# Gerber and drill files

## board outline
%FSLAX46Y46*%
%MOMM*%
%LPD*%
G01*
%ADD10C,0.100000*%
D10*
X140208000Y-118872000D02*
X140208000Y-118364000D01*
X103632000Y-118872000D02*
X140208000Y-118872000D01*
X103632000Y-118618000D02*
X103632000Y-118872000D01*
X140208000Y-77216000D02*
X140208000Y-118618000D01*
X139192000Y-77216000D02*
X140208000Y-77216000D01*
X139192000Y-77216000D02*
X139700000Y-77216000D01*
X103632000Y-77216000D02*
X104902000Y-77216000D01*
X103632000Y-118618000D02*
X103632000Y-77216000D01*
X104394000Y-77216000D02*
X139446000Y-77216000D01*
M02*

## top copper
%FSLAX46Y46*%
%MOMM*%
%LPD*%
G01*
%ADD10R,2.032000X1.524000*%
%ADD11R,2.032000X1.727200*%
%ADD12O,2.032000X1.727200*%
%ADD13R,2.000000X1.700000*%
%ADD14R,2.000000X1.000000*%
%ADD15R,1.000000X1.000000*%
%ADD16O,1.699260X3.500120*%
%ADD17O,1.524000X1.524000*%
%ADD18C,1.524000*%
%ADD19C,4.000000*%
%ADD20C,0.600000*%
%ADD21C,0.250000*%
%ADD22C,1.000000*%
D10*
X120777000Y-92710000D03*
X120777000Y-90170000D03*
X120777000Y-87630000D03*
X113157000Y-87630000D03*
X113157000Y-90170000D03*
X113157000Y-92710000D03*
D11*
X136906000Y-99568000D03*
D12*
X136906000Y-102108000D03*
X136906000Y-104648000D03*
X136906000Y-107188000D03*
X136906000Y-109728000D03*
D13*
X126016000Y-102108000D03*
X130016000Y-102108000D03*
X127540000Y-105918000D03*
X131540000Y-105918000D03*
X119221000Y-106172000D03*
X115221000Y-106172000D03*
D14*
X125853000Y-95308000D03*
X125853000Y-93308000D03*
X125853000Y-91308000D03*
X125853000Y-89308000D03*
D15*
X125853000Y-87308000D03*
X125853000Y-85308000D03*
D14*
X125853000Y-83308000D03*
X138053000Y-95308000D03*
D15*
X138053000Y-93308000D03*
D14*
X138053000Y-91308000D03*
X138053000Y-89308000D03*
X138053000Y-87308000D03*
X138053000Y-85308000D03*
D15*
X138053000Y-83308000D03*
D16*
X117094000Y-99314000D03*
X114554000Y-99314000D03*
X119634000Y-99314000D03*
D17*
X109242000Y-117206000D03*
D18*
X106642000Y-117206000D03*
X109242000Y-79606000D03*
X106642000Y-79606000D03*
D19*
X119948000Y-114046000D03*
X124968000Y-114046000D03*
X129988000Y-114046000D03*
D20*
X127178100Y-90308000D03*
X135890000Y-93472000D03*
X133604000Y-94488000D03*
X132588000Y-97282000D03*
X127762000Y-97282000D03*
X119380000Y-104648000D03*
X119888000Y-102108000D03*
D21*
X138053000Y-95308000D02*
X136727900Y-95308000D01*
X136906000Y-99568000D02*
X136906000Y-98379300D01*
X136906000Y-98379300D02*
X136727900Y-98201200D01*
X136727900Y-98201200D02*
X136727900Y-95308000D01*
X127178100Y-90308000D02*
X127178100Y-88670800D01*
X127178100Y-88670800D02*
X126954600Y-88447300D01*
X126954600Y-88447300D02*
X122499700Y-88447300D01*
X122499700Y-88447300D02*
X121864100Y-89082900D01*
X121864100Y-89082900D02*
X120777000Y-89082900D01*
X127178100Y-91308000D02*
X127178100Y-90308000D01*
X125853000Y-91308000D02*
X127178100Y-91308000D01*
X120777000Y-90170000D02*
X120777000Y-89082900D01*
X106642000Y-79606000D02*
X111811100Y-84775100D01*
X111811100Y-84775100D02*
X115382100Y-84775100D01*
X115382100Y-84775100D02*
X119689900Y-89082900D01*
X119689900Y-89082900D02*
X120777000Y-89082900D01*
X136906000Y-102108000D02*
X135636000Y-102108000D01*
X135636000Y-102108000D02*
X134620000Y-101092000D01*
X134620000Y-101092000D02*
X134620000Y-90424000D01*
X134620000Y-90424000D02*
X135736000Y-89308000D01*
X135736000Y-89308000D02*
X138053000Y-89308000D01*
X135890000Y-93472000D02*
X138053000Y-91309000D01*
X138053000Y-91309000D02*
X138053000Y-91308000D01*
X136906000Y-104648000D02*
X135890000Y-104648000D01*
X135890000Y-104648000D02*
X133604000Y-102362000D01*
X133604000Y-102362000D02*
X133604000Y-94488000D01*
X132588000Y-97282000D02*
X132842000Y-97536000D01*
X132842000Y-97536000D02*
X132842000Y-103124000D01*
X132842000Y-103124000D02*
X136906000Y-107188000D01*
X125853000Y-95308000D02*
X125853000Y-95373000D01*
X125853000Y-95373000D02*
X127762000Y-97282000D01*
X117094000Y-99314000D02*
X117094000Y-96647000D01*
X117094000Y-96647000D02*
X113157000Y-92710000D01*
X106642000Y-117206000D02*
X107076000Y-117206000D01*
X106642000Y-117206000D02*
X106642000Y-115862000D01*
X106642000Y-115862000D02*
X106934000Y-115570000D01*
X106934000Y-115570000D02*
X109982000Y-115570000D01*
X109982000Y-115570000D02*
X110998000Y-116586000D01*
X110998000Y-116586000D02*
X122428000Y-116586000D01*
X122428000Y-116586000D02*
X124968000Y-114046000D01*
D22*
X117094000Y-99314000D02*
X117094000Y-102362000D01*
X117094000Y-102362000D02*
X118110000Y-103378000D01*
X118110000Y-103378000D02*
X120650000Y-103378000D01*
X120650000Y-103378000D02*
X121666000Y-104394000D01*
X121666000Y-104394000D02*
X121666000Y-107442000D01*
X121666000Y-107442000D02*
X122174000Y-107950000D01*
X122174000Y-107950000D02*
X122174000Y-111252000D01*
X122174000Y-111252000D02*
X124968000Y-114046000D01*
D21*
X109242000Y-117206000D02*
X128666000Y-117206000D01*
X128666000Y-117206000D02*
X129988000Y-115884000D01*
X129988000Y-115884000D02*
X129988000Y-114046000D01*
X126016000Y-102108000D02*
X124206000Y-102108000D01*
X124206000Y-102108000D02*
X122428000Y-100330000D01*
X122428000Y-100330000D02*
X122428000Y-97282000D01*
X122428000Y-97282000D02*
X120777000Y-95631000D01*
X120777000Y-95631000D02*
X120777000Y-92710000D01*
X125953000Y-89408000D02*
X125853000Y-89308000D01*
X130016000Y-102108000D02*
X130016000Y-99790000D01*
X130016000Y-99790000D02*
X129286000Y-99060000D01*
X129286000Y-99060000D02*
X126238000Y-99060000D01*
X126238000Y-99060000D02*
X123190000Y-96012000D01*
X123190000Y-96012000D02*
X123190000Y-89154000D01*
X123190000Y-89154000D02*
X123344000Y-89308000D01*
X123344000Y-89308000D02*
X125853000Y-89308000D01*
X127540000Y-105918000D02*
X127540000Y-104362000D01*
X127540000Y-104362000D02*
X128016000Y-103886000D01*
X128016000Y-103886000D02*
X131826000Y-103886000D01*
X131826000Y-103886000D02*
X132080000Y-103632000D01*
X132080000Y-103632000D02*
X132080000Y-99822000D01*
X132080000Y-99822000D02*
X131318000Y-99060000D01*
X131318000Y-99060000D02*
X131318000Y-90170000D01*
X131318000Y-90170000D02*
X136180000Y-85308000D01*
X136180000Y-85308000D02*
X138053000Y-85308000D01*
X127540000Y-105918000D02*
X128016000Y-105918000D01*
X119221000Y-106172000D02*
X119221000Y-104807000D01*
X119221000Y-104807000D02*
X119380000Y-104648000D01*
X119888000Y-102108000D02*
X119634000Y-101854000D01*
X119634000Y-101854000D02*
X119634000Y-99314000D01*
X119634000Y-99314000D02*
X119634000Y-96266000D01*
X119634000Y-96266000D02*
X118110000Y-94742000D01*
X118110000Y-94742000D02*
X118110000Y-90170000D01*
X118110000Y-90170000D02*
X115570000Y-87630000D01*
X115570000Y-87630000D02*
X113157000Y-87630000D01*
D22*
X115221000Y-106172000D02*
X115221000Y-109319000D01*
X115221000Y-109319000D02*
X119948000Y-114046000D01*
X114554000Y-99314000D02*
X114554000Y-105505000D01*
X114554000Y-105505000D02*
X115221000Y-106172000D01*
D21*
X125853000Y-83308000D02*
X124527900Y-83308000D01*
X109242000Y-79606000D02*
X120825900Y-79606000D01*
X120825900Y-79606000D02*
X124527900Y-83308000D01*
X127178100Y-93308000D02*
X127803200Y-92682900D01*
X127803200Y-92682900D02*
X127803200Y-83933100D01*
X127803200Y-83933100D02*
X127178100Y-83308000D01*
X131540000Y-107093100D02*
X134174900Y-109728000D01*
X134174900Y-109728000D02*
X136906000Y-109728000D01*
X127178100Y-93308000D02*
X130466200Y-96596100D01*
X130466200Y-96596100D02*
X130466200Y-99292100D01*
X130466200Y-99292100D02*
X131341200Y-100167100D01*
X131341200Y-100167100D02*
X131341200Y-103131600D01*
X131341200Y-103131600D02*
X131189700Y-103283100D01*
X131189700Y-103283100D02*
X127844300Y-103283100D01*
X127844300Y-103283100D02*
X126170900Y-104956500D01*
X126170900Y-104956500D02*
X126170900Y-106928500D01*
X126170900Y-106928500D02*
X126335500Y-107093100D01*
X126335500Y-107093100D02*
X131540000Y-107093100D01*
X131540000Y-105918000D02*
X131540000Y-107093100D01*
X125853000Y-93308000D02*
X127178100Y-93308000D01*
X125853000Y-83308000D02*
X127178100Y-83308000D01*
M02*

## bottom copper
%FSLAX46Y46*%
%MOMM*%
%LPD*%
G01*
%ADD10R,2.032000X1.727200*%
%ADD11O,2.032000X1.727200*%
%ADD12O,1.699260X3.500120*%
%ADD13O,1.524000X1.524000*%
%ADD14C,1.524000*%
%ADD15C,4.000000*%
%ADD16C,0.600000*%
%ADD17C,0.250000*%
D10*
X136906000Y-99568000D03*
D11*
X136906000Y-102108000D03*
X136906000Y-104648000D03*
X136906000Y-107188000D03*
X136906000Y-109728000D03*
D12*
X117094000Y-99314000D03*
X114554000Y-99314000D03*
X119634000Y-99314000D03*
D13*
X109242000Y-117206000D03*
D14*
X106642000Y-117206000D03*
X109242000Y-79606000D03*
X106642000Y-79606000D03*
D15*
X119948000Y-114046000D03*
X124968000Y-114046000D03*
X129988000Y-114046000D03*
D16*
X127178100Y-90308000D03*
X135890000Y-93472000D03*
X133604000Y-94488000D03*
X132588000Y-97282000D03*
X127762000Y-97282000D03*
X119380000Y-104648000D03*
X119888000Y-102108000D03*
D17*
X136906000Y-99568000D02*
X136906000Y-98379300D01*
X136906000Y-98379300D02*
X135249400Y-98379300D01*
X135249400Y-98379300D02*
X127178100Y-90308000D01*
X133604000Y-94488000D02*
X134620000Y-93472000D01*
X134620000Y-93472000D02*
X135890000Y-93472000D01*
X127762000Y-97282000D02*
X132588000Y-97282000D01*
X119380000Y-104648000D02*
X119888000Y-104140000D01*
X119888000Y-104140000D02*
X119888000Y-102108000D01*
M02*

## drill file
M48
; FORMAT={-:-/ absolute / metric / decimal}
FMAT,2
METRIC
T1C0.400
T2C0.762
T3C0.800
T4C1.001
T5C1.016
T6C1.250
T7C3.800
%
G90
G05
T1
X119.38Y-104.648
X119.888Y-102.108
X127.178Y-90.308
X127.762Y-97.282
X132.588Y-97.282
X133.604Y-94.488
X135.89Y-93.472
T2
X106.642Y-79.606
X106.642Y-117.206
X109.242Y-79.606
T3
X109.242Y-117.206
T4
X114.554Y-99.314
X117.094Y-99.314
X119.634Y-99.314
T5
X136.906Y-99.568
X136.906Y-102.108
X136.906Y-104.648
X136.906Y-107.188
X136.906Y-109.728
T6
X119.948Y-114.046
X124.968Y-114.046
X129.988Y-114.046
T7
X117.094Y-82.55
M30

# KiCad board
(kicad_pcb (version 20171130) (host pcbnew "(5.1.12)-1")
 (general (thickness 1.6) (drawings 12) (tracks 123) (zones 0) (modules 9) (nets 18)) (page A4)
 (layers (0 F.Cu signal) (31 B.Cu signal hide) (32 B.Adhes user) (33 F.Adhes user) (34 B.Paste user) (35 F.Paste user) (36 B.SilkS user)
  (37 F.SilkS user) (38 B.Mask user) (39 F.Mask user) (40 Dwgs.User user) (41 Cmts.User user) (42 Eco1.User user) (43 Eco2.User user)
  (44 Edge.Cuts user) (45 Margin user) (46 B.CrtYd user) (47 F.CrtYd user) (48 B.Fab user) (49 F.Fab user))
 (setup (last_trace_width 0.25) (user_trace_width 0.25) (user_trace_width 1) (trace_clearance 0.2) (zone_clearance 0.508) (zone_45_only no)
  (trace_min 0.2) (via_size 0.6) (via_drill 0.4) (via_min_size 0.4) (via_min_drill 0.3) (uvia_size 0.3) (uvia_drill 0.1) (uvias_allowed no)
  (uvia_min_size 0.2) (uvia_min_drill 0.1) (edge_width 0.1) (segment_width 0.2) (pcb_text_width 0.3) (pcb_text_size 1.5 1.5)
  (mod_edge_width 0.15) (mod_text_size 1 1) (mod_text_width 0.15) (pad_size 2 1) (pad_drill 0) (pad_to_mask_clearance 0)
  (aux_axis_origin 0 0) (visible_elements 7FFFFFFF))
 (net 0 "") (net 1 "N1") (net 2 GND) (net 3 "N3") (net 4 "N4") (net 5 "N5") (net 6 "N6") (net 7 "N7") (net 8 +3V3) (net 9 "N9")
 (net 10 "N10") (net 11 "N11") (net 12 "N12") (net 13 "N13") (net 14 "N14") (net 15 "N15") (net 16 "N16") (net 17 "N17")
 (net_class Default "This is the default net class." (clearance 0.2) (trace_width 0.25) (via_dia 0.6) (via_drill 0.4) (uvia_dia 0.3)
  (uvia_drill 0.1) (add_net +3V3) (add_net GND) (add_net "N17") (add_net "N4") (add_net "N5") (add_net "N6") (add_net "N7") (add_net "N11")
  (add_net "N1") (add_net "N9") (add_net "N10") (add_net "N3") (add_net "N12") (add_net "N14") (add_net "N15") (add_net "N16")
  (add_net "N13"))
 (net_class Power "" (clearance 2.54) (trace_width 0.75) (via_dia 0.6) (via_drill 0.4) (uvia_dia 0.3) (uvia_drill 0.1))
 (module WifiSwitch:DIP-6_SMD (layer F.Cu) (at 116.967 88.9 90)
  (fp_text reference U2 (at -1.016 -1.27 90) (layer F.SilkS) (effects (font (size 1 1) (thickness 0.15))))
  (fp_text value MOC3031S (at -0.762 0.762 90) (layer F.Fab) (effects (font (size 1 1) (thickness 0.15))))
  (pad 1 smd rect (at -3.81 3.81 90) (size 1.524 2.032) (layers F.Cu F.Paste F.Mask) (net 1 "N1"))
  (pad 2 smd rect (at -1.27 3.81 90) (size 1.524 2.032) (layers F.Cu F.Paste F.Mask) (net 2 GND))
  (pad 3 smd rect (at 1.27 3.81 90) (size 1.524 2.032) (layers F.Cu F.Paste F.Mask))
  (pad 4 smd rect (at 1.27 -3.81 90) (size 1.524 2.032) (layers F.Cu F.Paste F.Mask) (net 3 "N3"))
  (pad 5 smd rect (at -1.27 -3.81 90) (size 1.524 2.032) (layers F.Cu F.Paste F.Mask))
  (pad 6 smd rect (at -3.81 -3.81 90) (size 1.524 2.032) (layers F.Cu F.Paste F.Mask) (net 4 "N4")))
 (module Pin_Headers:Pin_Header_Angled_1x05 (layer F.Cu) (at 136.906 99.568)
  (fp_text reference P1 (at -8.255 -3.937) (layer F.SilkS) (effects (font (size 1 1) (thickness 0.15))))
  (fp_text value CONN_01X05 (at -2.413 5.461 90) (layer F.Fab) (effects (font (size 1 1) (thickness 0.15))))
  (pad 1 thru_hole rect (at 0 0) (size 2.032 1.7272) (drill 1.016) (layers *.Cu *.Mask F.SilkS) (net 2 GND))
  (pad 2 thru_hole oval (at 0 2.54) (size 2.032 1.7272) (drill 1.016) (layers *.Cu *.Mask F.SilkS) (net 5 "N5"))
  (pad 3 thru_hole oval (at 0 5.08) (size 2.032 1.7272) (drill 1.016) (layers *.Cu *.Mask F.SilkS) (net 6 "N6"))
  (pad 4 thru_hole oval (at 0 7.62) (size 2.032 1.7272) (drill 1.016) (layers *.Cu *.Mask F.SilkS) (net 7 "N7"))
  (pad 5 thru_hole oval (at 0 10.16) (size 2.032 1.7272) (drill 1.016) (layers *.Cu *.Mask F.SilkS) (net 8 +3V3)))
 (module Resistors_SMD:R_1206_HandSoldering (layer F.Cu) (at 128.016 102.108)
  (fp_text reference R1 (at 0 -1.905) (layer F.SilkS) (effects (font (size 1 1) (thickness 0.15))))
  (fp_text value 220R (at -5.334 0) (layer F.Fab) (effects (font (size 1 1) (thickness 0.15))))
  (pad 1 smd rect (at -2 0) (size 2 1.7) (layers F.Cu F.Paste F.Mask) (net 1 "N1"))
  (pad 2 smd rect (at 2 0) (size 2 1.7) (layers F.Cu F.Paste F.Mask) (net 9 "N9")))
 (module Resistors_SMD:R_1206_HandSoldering (layer F.Cu) (at 129.54 105.918)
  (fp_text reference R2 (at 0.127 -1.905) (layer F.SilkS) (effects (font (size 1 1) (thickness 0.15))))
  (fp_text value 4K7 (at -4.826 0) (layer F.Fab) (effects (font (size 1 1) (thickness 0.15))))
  (pad 1 smd rect (at -2 0) (size 2 1.7) (layers F.Cu F.Paste F.Mask) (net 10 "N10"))
  (pad 2 smd rect (at 2 0) (size 2 1.7) (layers F.Cu F.Paste F.Mask) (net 8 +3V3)))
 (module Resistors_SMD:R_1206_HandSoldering (layer F.Cu) (at 117.221 106.172 180)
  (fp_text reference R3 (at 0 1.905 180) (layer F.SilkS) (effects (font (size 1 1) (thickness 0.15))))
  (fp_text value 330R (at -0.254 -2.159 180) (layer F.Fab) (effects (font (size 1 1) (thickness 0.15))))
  (pad 1 smd rect (at -2 0 180) (size 2 1.7) (layers F.Cu F.Paste F.Mask) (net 3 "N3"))
  (pad 2 smd rect (at 2 0 180) (size 2 1.7) (layers F.Cu F.Paste F.Mask) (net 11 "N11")))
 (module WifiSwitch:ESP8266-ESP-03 (layer F.Cu) (at 131.953 89.408)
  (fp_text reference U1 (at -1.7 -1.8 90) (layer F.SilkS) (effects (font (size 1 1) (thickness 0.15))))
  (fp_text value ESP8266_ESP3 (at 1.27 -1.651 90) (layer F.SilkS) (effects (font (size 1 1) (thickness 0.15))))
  (pad 14 smd rect (at -6.1 5.9) (size 2 1) (layers F.Cu F.Paste F.Mask) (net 7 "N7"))
  (pad 13 smd rect (at -6.1 3.9) (size 2 1) (layers F.Cu F.Paste F.Mask) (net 8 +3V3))
  (pad 12 smd rect (at -6.1 1.9) (size 2 1) (layers F.Cu F.Paste F.Mask) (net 2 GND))
  (pad 11 smd rect (at -6.1 -0.1) (size 2 1) (layers F.Cu F.Paste F.Mask) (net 9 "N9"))
  (pad 10 smd rect (at -6.1 -2.1) (size 1 1) (layers F.Cu F.Paste F.Mask) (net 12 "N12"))
  (pad 9 smd rect (at -6.1 -4.1) (size 1 1) (layers F.Cu F.Paste F.Mask) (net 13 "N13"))
  (pad 8 smd rect (at -6.1 -6.1) (size 2 1) (layers F.Cu F.Paste F.Mask) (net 8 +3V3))
  (pad 1 smd rect (at 6.1 5.9) (size 2 1) (layers F.Cu F.Paste F.Mask) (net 2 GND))
  (pad 2 smd rect (at 6.1 3.9) (size 1 1) (layers F.Cu F.Paste F.Mask) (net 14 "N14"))
  (pad 3 smd rect (at 6.1 1.9) (size 2 1) (layers F.Cu F.Paste F.Mask) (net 6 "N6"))
  (pad 4 smd rect (at 6.1 -0.1) (size 2 1) (layers F.Cu F.Paste F.Mask) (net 5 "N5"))
  (pad 5 smd rect (at 6.1 -2.1) (size 2 1) (layers F.Cu F.Paste F.Mask) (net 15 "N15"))
  (pad 6 smd rect (at 6.1 -4.1) (size 2 1) (layers F.Cu F.Paste F.Mask) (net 10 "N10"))
  (pad 7 smd rect (at 6.1 -6.1) (size 1 1) (layers F.Cu F.Paste F.Mask) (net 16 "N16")))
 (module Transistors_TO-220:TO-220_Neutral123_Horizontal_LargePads (layer F.Cu) (at 117.094 99.314)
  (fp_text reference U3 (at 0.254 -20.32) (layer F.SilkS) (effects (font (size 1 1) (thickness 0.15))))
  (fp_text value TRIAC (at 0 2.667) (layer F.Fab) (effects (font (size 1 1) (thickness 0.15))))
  (pad 2 thru_hole oval (at 0 0 90) (size 3.50012 1.69926) (drill 1.00076) (layers *.Cu *.Mask F.SilkS) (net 4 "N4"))
  (pad 1 thru_hole oval (at -2.54 0 90) (size 3.50012 1.69926) (drill 1.00076) (layers *.Cu *.Mask F.SilkS) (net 11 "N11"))
  (pad 3 thru_hole oval (at 2.54 0 90) (size 3.50012 1.69926) (drill 1.00076) (layers *.Cu *.Mask F.SilkS) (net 3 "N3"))
  (pad "" np_thru_hole circle (at 0 -16.764 90) (size 3.79984 3.79984) (drill 3.79984) (layers *.Cu *.Mask F.SilkS)))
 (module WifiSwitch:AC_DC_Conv (layer F.Cu) (at 107.442 98.806 270)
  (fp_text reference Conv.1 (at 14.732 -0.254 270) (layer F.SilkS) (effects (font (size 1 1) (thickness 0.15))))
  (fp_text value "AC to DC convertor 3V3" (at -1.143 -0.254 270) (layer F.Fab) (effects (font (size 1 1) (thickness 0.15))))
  (pad 3 thru_hole oval (at 18.4 -1.8 270) (size 1.524 1.524) (drill 0.8) (layers *.Cu *.Mask F.SilkS) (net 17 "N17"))
  (pad 4 thru_hole circle (at 18.4 0.8 270) (size 1.524 1.524) (drill 0.762) (layers *.Cu *.Mask F.SilkS) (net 4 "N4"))
  (pad 1 thru_hole circle (at -19.2 -1.8 270) (size 1.524 1.524) (drill 0.762) (layers *.Cu *.Mask F.SilkS) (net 8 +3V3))
  (pad 2 thru_hole circle (at -19.2 0.8 270) (size 1.524 1.524) (drill 0.762) (layers *.Cu *.Mask F.SilkS) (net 2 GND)))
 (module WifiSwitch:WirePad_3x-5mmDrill (layer F.Cu) (at 124.968 114.046)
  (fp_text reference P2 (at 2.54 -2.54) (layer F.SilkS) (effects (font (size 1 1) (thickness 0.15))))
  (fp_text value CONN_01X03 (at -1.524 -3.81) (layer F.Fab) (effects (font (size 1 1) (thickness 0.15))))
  (pad 1 thru_hole circle (at -5.02 0) (size 4 4) (drill 1.25) (layers *.Cu *.Mask F.SilkS) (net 11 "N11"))
  (pad 2 thru_hole circle (at 0 0) (size 4 4) (drill 1.25) (layers *.Cu *.Mask F.SilkS) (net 4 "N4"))
  (pad 3 thru_hole circle (at 5.02 0) (size 4 4) (drill 1.25) (layers *.Cu *.Mask F.SilkS) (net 17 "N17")))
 (gr_line (start 140.208 118.872) (end 140.208 118.364) (angle 90) (layer Edge.Cuts) (width 0.1))
 (gr_line (start 103.632 118.872) (end 140.208 118.872) (angle 90) (layer Edge.Cuts) (width 0.1))
 (gr_line (start 103.632 118.618) (end 103.632 118.872) (angle 90) (layer Edge.Cuts) (width 0.1))
 (gr_line (start 140.208 77.216) (end 140.208 118.618) (angle 90) (layer Edge.Cuts) (width 0.1))
 (gr_line (start 139.192 77.216) (end 140.208 77.216) (angle 90) (layer Edge.Cuts) (width 0.1))
 (gr_line (start 139.192 77.216) (end 139.7 77.216) (angle 90) (layer Edge.Cuts) (width 0.1))
 (gr_line (start 103.632 77.216) (end 104.902 77.216) (angle 90) (layer Edge.Cuts) (width 0.1))
 (gr_line (start 103.632 118.618) (end 103.632 77.216) (angle 90) (layer Edge.Cuts) (width 0.1))
 (gr_line (start 104.394 77.216) (end 139.446 77.216) (angle 90) (layer Edge.Cuts) (width 0.1))
 (segment (start 138.053 95.308) (end 136.7279 95.308) (width 0.25) (layer F.Cu) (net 2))
 (segment (start 136.906 99.568) (end 136.906 98.3793) (width 0.25) (layer F.Cu) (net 2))
 (segment (start 136.906 98.3793) (end 136.7279 98.2012) (width 0.25) (layer F.Cu) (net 2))
 (segment (start 136.7279 98.2012) (end 136.7279 95.308) (width 0.25) (layer F.Cu) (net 2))
 (segment (start 136.906 99.568) (end 136.906 98.3793) (width 0.25) (layer B.Cu) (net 2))
 (segment (start 127.1781 90.308) (end 127.1781 88.6708) (width 0.25) (layer F.Cu) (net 2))
 (segment (start 127.1781 88.6708) (end 126.9546 88.4473) (width 0.25) (layer F.Cu) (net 2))
 (segment (start 126.9546 88.4473) (end 122.4997 88.4473) (width 0.25) (layer F.Cu) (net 2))
 (segment (start 122.4997 88.4473) (end 121.8641 89.0829) (width 0.25) (layer F.Cu) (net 2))
 (segment (start 121.8641 89.0829) (end 120.777 89.0829) (width 0.25) (layer F.Cu) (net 2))
 (segment (start 127.1781 91.308) (end 127.1781 90.308) (width 0.25) (layer F.Cu) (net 2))
 (segment (start 136.906 98.3793) (end 135.2494 98.3793) (width 0.25) (layer B.Cu) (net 2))
 (segment (start 135.2494 98.3793) (end 127.1781 90.308) (width 0.25) (layer B.Cu) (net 2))
 (segment (start 125.853 91.308) (end 127.1781 91.308) (width 0.25) (layer F.Cu) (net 2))
 (segment (start 120.777 90.17) (end 120.777 89.0829) (width 0.25) (layer F.Cu) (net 2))
 (segment (start 106.642 79.606) (end 111.8111 84.7751) (width 0.25) (layer F.Cu) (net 2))
 (segment (start 111.8111 84.7751) (end 115.3821 84.7751) (width 0.25) (layer F.Cu) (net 2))
 (segment (start 115.3821 84.7751) (end 119.6899 89.0829) (width 0.25) (layer F.Cu) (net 2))
 (segment (start 119.6899 89.0829) (end 120.777 89.0829) (width 0.25) (layer F.Cu) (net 2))
 (via (at 127.1781 90.308) (size 0.6) (layers F.Cu B.Cu) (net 2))
 (segment (start 136.906 102.108) (end 135.636 102.108) (width 0.25) (layer F.Cu) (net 5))
 (segment (start 135.636 102.108) (end 134.62 101.092) (width 0.25) (layer F.Cu) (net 5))
 (segment (start 134.62 101.092) (end 134.62 90.424) (width 0.25) (layer F.Cu) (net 5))
 (segment (start 134.62 90.424) (end 135.736 89.308) (width 0.25) (layer F.Cu) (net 5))
 (segment (start 135.736 89.308) (end 138.053 89.308) (width 0.25) (layer F.Cu) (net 5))
 (segment (start 135.89 93.472) (end 138.053 91.309) (width 0.25) (layer F.Cu) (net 6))
 (segment (start 138.053 91.309) (end 138.053 91.308) (width 0.25) (layer F.Cu) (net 6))
 (segment (start 133.604 94.488) (end 134.62 93.472) (width 0.25) (layer B.Cu) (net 6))
 (segment (start 134.62 93.472) (end 135.89 93.472) (width 0.25) (layer B.Cu) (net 6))
 (segment (start 136.906 104.648) (end 135.89 104.648) (width 0.25) (layer F.Cu) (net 6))
 (segment (start 135.89 104.648) (end 133.604 102.362) (width 0.25) (layer F.Cu) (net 6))
 (segment (start 133.604 102.362) (end 133.604 94.488) (width 0.25) (layer F.Cu) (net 6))
 (via (at 135.89 93.472) (size 0.6) (layers F.Cu B.Cu) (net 6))
 (via (at 133.604 94.488) (size 0.6) (layers F.Cu B.Cu) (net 6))
 (segment (start 132.588 97.282) (end 132.842 97.536) (width 0.25) (layer F.Cu) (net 7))
 (segment (start 132.842 97.536) (end 132.842 103.124) (width 0.25) (layer F.Cu) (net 7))
 (segment (start 132.842 103.124) (end 136.906 107.188) (width 0.25) (layer F.Cu) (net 7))
 (segment (start 127.762 97.282) (end 132.588 97.282) (width 0.25) (layer B.Cu) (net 7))
 (segment (start 125.853 95.308) (end 125.853 95.373) (width 0.25) (layer F.Cu) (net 7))
 (segment (start 125.853 95.373) (end 127.762 97.282) (width 0.25) (layer F.Cu) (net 7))
 (via (at 132.588 97.282) (size 0.6) (layers F.Cu B.Cu) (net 7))
 (via (at 127.762 97.282) (size 0.6) (layers F.Cu B.Cu) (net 7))
 (segment (start 117.094 99.314) (end 117.094 96.647) (width 0.25) (layer F.Cu) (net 4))
 (segment (start 117.094 96.647) (end 113.157 92.71) (width 0.25) (layer F.Cu) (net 4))
 (segment (start 106.642 117.206) (end 107.076 117.206) (width 0.25) (layer F.Cu) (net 4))
 (segment (start 106.642 117.206) (end 106.642 115.862) (width 0.25) (layer F.Cu) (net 4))
 (segment (start 106.642 115.862) (end 106.934 115.57) (width 0.25) (layer F.Cu) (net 4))
 (segment (start 106.934 115.57) (end 109.982 115.57) (width 0.25) (layer F.Cu) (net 4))
 (segment (start 109.982 115.57) (end 110.998 116.586) (width 0.25) (layer F.Cu) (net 4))
 (segment (start 110.998 116.586) (end 122.428 116.586) (width 0.25) (layer F.Cu) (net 4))
 (segment (start 122.428 116.586) (end 124.968 114.046) (width 0.25) (layer F.Cu) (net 4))
 (segment (start 117.094 99.314) (end 117.094 102.362) (width 1) (layer F.Cu) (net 4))
 (segment (start 117.094 102.362) (end 118.11 103.378) (width 1) (layer F.Cu) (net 4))
 (segment (start 118.11 103.378) (end 120.65 103.378) (width 1) (layer F.Cu) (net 4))
 (segment (start 120.65 103.378) (end 121.666 104.394) (width 1) (layer F.Cu) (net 4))
 (segment (start 121.666 104.394) (end 121.666 107.442) (width 1) (layer F.Cu) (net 4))
 (segment (start 121.666 107.442) (end 122.174 107.95) (width 1) (layer F.Cu) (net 4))
 (segment (start 122.174 107.95) (end 122.174 111.252) (width 1) (layer F.Cu) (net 4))
 (segment (start 122.174 111.252) (end 124.968 114.046) (width 1) (layer F.Cu) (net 4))
 (segment (start 109.242 117.206) (end 128.666 117.206) (width 0.25) (layer F.Cu) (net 17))
 (segment (start 128.666 117.206) (end 129.988 115.884) (width 0.25) (layer F.Cu) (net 17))
 (segment (start 129.988 115.884) (end 129.988 114.046) (width 0.25) (layer F.Cu) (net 17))
 (segment (start 126.016 102.108) (end 124.206 102.108) (width 0.25) (layer F.Cu) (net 1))
 (segment (start 124.206 102.108) (end 122.428 100.33) (width 0.25) (layer F.Cu) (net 1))
 (segment (start 122.428 100.33) (end 122.428 97.282) (width 0.25) (layer F.Cu) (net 1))
 (segment (start 122.428 97.282) (end 120.777 95.631) (width 0.25) (layer F.Cu) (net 1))
 (segment (start 120.777 95.631) (end 120.777 92.71) (width 0.25) (layer F.Cu) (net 1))
 (segment (start 125.953 89.408) (end 125.853 89.308) (width 0.25) (layer F.Cu) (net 9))
 (segment (start 130.016 102.108) (end 130.016 99.79) (width 0.25) (layer F.Cu) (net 9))
 (segment (start 130.016 99.79) (end 129.286 99.06) (width 0.25) (layer F.Cu) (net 9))
 (segment (start 129.286 99.06) (end 126.238 99.06) (width 0.25) (layer F.Cu) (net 9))
 (segment (start 126.238 99.06) (end 123.19 96.012) (width 0.25) (layer F.Cu) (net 9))
 (segment (start 123.19 96.012) (end 123.19 89.154) (width 0.25) (layer F.Cu) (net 9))
 (segment (start 123.19 89.154) (end 123.344 89.308) (width 0.25) (layer F.Cu) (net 9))
 (segment (start 123.344 89.308) (end 125.853 89.308) (width 0.25) (layer F.Cu) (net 9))
 (segment (start 127.54 105.918) (end 127.54 104.362) (width 0.25) (layer F.Cu) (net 10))
 (segment (start 127.54 104.362) (end 128.016 103.886) (width 0.25) (layer F.Cu) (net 10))
 (segment (start 128.016 103.886) (end 131.826 103.886) (width 0.25) (layer F.Cu) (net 10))
 (segment (start 131.826 103.886) (end 132.08 103.632) (width 0.25) (layer F.Cu) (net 10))
 (segment (start 132.08 103.632) (end 132.08 99.822) (width 0.25) (layer F.Cu) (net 10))
 (segment (start 132.08 99.822) (end 131.318 99.06) (width 0.25) (layer F.Cu) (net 10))
 (segment (start 131.318 99.06) (end 131.318 90.17) (width 0.25) (layer F.Cu) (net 10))
 (segment (start 131.318 90.17) (end 136.18 85.308) (width 0.25) (layer F.Cu) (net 10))
 (segment (start 136.18 85.308) (end 138.053 85.308) (width 0.25) (layer F.Cu) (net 10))
 (segment (start 127.54 105.918) (end 128.016 105.918) (width 0.25) (layer F.Cu) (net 10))
 (segment (start 119.221 106.172) (end 119.221 104.807) (width 0.25) (layer F.Cu) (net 3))
 (segment (start 119.221 104.807) (end 119.38 104.648) (width 0.25) (layer F.Cu) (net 3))
 (segment (start 119.38 104.648) (end 119.888 104.14) (width 0.25) (layer B.Cu) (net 3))
 (segment (start 119.888 104.14) (end 119.888 102.108) (width 0.25) (layer B.Cu) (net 3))
 (segment (start 119.888 102.108) (end 119.634 101.854) (width 0.25) (layer F.Cu) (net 3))
 (segment (start 119.634 101.854) (end 119.634 99.314) (width 0.25) (layer F.Cu) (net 3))
 (segment (start 119.634 99.314) (end 119.634 96.266) (width 0.25) (layer F.Cu) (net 3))
 (segment (start 119.634 96.266) (end 118.11 94.742) (width 0.25) (layer F.Cu) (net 3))
 (segment (start 118.11 94.742) (end 118.11 90.17) (width 0.25) (layer F.Cu) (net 3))
 (segment (start 118.11 90.17) (end 115.57 87.63) (width 0.25) (layer F.Cu) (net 3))
 (segment (start 115.57 87.63) (end 113.157 87.63) (width 0.25) (layer F.Cu) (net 3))
 (via (at 119.38 104.648) (size 0.6) (layers F.Cu B.Cu) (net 3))
 (via (at 119.888 102.108) (size 0.6) (layers F.Cu B.Cu) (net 3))
 (segment (start 115.221 106.172) (end 115.221 109.319) (width 1) (layer F.Cu) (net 11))
 (segment (start 115.221 109.319) (end 119.948 114.046) (width 1) (layer F.Cu) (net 11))
 (segment (start 114.554 99.314) (end 114.554 105.505) (width 1) (layer F.Cu) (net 11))
 (segment (start 114.554 105.505) (end 115.221 106.172) (width 1) (layer F.Cu) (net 11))
 (segment (start 125.853 83.308) (end 124.5279 83.308) (width 0.25) (layer F.Cu) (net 8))
 (segment (start 109.242 79.606) (end 120.8259 79.606) (width 0.25) (layer F.Cu) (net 8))
 (segment (start 120.8259 79.606) (end 124.5279 83.308) (width 0.25) (layer F.Cu) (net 8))
 (segment (start 127.1781 93.308) (end 127.8032 92.6829) (width 0.25) (layer F.Cu) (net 8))
 (segment (start 127.8032 92.6829) (end 127.8032 83.9331) (width 0.25) (layer F.Cu) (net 8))
 (segment (start 127.8032 83.9331) (end 127.1781 83.308) (width 0.25) (layer F.Cu) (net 8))
 (segment (start 131.54 107.0931) (end 134.1749 109.728) (width 0.25) (layer F.Cu) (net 8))
 (segment (start 134.1749 109.728) (end 136.906 109.728) (width 0.25) (layer F.Cu) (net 8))
 (segment (start 127.1781 93.308) (end 130.4662 96.5961) (width 0.25) (layer F.Cu) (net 8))
 (segment (start 130.4662 96.5961) (end 130.4662 99.2921) (width 0.25) (layer F.Cu) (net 8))
 (segment (start 130.4662 99.2921) (end 131.3412 100.1671) (width 0.25) (layer F.Cu) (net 8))
 (segment (start 131.3412 100.1671) (end 131.3412 103.1316) (width 0.25) (layer F.Cu) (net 8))
 (segment (start 131.3412 103.1316) (end 131.1897 103.2831) (width 0.25) (layer F.Cu) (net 8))
 (segment (start 131.1897 103.2831) (end 127.8443 103.2831) (width 0.25) (layer F.Cu) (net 8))
 (segment (start 127.8443 103.2831) (end 126.1709 104.9565) (width 0.25) (layer F.Cu) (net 8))
 (segment (start 126.1709 104.9565) (end 126.1709 106.9285) (width 0.25) (layer F.Cu) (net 8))
 (segment (start 126.1709 106.9285) (end 126.3355 107.0931) (width 0.25) (layer F.Cu) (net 8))
 (segment (start 126.3355 107.0931) (end 131.54 107.0931) (width 0.25) (layer F.Cu) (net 8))
 (segment (start 131.54 105.918) (end 131.54 107.0931) (width 0.25) (layer F.Cu) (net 8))
 (segment (start 125.853 93.308) (end 127.1781 93.308) (width 0.25) (layer F.Cu) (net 8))
 (segment (start 125.853 83.308) (end 127.1781 83.308) (width 0.25) (layer F.Cu) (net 8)))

